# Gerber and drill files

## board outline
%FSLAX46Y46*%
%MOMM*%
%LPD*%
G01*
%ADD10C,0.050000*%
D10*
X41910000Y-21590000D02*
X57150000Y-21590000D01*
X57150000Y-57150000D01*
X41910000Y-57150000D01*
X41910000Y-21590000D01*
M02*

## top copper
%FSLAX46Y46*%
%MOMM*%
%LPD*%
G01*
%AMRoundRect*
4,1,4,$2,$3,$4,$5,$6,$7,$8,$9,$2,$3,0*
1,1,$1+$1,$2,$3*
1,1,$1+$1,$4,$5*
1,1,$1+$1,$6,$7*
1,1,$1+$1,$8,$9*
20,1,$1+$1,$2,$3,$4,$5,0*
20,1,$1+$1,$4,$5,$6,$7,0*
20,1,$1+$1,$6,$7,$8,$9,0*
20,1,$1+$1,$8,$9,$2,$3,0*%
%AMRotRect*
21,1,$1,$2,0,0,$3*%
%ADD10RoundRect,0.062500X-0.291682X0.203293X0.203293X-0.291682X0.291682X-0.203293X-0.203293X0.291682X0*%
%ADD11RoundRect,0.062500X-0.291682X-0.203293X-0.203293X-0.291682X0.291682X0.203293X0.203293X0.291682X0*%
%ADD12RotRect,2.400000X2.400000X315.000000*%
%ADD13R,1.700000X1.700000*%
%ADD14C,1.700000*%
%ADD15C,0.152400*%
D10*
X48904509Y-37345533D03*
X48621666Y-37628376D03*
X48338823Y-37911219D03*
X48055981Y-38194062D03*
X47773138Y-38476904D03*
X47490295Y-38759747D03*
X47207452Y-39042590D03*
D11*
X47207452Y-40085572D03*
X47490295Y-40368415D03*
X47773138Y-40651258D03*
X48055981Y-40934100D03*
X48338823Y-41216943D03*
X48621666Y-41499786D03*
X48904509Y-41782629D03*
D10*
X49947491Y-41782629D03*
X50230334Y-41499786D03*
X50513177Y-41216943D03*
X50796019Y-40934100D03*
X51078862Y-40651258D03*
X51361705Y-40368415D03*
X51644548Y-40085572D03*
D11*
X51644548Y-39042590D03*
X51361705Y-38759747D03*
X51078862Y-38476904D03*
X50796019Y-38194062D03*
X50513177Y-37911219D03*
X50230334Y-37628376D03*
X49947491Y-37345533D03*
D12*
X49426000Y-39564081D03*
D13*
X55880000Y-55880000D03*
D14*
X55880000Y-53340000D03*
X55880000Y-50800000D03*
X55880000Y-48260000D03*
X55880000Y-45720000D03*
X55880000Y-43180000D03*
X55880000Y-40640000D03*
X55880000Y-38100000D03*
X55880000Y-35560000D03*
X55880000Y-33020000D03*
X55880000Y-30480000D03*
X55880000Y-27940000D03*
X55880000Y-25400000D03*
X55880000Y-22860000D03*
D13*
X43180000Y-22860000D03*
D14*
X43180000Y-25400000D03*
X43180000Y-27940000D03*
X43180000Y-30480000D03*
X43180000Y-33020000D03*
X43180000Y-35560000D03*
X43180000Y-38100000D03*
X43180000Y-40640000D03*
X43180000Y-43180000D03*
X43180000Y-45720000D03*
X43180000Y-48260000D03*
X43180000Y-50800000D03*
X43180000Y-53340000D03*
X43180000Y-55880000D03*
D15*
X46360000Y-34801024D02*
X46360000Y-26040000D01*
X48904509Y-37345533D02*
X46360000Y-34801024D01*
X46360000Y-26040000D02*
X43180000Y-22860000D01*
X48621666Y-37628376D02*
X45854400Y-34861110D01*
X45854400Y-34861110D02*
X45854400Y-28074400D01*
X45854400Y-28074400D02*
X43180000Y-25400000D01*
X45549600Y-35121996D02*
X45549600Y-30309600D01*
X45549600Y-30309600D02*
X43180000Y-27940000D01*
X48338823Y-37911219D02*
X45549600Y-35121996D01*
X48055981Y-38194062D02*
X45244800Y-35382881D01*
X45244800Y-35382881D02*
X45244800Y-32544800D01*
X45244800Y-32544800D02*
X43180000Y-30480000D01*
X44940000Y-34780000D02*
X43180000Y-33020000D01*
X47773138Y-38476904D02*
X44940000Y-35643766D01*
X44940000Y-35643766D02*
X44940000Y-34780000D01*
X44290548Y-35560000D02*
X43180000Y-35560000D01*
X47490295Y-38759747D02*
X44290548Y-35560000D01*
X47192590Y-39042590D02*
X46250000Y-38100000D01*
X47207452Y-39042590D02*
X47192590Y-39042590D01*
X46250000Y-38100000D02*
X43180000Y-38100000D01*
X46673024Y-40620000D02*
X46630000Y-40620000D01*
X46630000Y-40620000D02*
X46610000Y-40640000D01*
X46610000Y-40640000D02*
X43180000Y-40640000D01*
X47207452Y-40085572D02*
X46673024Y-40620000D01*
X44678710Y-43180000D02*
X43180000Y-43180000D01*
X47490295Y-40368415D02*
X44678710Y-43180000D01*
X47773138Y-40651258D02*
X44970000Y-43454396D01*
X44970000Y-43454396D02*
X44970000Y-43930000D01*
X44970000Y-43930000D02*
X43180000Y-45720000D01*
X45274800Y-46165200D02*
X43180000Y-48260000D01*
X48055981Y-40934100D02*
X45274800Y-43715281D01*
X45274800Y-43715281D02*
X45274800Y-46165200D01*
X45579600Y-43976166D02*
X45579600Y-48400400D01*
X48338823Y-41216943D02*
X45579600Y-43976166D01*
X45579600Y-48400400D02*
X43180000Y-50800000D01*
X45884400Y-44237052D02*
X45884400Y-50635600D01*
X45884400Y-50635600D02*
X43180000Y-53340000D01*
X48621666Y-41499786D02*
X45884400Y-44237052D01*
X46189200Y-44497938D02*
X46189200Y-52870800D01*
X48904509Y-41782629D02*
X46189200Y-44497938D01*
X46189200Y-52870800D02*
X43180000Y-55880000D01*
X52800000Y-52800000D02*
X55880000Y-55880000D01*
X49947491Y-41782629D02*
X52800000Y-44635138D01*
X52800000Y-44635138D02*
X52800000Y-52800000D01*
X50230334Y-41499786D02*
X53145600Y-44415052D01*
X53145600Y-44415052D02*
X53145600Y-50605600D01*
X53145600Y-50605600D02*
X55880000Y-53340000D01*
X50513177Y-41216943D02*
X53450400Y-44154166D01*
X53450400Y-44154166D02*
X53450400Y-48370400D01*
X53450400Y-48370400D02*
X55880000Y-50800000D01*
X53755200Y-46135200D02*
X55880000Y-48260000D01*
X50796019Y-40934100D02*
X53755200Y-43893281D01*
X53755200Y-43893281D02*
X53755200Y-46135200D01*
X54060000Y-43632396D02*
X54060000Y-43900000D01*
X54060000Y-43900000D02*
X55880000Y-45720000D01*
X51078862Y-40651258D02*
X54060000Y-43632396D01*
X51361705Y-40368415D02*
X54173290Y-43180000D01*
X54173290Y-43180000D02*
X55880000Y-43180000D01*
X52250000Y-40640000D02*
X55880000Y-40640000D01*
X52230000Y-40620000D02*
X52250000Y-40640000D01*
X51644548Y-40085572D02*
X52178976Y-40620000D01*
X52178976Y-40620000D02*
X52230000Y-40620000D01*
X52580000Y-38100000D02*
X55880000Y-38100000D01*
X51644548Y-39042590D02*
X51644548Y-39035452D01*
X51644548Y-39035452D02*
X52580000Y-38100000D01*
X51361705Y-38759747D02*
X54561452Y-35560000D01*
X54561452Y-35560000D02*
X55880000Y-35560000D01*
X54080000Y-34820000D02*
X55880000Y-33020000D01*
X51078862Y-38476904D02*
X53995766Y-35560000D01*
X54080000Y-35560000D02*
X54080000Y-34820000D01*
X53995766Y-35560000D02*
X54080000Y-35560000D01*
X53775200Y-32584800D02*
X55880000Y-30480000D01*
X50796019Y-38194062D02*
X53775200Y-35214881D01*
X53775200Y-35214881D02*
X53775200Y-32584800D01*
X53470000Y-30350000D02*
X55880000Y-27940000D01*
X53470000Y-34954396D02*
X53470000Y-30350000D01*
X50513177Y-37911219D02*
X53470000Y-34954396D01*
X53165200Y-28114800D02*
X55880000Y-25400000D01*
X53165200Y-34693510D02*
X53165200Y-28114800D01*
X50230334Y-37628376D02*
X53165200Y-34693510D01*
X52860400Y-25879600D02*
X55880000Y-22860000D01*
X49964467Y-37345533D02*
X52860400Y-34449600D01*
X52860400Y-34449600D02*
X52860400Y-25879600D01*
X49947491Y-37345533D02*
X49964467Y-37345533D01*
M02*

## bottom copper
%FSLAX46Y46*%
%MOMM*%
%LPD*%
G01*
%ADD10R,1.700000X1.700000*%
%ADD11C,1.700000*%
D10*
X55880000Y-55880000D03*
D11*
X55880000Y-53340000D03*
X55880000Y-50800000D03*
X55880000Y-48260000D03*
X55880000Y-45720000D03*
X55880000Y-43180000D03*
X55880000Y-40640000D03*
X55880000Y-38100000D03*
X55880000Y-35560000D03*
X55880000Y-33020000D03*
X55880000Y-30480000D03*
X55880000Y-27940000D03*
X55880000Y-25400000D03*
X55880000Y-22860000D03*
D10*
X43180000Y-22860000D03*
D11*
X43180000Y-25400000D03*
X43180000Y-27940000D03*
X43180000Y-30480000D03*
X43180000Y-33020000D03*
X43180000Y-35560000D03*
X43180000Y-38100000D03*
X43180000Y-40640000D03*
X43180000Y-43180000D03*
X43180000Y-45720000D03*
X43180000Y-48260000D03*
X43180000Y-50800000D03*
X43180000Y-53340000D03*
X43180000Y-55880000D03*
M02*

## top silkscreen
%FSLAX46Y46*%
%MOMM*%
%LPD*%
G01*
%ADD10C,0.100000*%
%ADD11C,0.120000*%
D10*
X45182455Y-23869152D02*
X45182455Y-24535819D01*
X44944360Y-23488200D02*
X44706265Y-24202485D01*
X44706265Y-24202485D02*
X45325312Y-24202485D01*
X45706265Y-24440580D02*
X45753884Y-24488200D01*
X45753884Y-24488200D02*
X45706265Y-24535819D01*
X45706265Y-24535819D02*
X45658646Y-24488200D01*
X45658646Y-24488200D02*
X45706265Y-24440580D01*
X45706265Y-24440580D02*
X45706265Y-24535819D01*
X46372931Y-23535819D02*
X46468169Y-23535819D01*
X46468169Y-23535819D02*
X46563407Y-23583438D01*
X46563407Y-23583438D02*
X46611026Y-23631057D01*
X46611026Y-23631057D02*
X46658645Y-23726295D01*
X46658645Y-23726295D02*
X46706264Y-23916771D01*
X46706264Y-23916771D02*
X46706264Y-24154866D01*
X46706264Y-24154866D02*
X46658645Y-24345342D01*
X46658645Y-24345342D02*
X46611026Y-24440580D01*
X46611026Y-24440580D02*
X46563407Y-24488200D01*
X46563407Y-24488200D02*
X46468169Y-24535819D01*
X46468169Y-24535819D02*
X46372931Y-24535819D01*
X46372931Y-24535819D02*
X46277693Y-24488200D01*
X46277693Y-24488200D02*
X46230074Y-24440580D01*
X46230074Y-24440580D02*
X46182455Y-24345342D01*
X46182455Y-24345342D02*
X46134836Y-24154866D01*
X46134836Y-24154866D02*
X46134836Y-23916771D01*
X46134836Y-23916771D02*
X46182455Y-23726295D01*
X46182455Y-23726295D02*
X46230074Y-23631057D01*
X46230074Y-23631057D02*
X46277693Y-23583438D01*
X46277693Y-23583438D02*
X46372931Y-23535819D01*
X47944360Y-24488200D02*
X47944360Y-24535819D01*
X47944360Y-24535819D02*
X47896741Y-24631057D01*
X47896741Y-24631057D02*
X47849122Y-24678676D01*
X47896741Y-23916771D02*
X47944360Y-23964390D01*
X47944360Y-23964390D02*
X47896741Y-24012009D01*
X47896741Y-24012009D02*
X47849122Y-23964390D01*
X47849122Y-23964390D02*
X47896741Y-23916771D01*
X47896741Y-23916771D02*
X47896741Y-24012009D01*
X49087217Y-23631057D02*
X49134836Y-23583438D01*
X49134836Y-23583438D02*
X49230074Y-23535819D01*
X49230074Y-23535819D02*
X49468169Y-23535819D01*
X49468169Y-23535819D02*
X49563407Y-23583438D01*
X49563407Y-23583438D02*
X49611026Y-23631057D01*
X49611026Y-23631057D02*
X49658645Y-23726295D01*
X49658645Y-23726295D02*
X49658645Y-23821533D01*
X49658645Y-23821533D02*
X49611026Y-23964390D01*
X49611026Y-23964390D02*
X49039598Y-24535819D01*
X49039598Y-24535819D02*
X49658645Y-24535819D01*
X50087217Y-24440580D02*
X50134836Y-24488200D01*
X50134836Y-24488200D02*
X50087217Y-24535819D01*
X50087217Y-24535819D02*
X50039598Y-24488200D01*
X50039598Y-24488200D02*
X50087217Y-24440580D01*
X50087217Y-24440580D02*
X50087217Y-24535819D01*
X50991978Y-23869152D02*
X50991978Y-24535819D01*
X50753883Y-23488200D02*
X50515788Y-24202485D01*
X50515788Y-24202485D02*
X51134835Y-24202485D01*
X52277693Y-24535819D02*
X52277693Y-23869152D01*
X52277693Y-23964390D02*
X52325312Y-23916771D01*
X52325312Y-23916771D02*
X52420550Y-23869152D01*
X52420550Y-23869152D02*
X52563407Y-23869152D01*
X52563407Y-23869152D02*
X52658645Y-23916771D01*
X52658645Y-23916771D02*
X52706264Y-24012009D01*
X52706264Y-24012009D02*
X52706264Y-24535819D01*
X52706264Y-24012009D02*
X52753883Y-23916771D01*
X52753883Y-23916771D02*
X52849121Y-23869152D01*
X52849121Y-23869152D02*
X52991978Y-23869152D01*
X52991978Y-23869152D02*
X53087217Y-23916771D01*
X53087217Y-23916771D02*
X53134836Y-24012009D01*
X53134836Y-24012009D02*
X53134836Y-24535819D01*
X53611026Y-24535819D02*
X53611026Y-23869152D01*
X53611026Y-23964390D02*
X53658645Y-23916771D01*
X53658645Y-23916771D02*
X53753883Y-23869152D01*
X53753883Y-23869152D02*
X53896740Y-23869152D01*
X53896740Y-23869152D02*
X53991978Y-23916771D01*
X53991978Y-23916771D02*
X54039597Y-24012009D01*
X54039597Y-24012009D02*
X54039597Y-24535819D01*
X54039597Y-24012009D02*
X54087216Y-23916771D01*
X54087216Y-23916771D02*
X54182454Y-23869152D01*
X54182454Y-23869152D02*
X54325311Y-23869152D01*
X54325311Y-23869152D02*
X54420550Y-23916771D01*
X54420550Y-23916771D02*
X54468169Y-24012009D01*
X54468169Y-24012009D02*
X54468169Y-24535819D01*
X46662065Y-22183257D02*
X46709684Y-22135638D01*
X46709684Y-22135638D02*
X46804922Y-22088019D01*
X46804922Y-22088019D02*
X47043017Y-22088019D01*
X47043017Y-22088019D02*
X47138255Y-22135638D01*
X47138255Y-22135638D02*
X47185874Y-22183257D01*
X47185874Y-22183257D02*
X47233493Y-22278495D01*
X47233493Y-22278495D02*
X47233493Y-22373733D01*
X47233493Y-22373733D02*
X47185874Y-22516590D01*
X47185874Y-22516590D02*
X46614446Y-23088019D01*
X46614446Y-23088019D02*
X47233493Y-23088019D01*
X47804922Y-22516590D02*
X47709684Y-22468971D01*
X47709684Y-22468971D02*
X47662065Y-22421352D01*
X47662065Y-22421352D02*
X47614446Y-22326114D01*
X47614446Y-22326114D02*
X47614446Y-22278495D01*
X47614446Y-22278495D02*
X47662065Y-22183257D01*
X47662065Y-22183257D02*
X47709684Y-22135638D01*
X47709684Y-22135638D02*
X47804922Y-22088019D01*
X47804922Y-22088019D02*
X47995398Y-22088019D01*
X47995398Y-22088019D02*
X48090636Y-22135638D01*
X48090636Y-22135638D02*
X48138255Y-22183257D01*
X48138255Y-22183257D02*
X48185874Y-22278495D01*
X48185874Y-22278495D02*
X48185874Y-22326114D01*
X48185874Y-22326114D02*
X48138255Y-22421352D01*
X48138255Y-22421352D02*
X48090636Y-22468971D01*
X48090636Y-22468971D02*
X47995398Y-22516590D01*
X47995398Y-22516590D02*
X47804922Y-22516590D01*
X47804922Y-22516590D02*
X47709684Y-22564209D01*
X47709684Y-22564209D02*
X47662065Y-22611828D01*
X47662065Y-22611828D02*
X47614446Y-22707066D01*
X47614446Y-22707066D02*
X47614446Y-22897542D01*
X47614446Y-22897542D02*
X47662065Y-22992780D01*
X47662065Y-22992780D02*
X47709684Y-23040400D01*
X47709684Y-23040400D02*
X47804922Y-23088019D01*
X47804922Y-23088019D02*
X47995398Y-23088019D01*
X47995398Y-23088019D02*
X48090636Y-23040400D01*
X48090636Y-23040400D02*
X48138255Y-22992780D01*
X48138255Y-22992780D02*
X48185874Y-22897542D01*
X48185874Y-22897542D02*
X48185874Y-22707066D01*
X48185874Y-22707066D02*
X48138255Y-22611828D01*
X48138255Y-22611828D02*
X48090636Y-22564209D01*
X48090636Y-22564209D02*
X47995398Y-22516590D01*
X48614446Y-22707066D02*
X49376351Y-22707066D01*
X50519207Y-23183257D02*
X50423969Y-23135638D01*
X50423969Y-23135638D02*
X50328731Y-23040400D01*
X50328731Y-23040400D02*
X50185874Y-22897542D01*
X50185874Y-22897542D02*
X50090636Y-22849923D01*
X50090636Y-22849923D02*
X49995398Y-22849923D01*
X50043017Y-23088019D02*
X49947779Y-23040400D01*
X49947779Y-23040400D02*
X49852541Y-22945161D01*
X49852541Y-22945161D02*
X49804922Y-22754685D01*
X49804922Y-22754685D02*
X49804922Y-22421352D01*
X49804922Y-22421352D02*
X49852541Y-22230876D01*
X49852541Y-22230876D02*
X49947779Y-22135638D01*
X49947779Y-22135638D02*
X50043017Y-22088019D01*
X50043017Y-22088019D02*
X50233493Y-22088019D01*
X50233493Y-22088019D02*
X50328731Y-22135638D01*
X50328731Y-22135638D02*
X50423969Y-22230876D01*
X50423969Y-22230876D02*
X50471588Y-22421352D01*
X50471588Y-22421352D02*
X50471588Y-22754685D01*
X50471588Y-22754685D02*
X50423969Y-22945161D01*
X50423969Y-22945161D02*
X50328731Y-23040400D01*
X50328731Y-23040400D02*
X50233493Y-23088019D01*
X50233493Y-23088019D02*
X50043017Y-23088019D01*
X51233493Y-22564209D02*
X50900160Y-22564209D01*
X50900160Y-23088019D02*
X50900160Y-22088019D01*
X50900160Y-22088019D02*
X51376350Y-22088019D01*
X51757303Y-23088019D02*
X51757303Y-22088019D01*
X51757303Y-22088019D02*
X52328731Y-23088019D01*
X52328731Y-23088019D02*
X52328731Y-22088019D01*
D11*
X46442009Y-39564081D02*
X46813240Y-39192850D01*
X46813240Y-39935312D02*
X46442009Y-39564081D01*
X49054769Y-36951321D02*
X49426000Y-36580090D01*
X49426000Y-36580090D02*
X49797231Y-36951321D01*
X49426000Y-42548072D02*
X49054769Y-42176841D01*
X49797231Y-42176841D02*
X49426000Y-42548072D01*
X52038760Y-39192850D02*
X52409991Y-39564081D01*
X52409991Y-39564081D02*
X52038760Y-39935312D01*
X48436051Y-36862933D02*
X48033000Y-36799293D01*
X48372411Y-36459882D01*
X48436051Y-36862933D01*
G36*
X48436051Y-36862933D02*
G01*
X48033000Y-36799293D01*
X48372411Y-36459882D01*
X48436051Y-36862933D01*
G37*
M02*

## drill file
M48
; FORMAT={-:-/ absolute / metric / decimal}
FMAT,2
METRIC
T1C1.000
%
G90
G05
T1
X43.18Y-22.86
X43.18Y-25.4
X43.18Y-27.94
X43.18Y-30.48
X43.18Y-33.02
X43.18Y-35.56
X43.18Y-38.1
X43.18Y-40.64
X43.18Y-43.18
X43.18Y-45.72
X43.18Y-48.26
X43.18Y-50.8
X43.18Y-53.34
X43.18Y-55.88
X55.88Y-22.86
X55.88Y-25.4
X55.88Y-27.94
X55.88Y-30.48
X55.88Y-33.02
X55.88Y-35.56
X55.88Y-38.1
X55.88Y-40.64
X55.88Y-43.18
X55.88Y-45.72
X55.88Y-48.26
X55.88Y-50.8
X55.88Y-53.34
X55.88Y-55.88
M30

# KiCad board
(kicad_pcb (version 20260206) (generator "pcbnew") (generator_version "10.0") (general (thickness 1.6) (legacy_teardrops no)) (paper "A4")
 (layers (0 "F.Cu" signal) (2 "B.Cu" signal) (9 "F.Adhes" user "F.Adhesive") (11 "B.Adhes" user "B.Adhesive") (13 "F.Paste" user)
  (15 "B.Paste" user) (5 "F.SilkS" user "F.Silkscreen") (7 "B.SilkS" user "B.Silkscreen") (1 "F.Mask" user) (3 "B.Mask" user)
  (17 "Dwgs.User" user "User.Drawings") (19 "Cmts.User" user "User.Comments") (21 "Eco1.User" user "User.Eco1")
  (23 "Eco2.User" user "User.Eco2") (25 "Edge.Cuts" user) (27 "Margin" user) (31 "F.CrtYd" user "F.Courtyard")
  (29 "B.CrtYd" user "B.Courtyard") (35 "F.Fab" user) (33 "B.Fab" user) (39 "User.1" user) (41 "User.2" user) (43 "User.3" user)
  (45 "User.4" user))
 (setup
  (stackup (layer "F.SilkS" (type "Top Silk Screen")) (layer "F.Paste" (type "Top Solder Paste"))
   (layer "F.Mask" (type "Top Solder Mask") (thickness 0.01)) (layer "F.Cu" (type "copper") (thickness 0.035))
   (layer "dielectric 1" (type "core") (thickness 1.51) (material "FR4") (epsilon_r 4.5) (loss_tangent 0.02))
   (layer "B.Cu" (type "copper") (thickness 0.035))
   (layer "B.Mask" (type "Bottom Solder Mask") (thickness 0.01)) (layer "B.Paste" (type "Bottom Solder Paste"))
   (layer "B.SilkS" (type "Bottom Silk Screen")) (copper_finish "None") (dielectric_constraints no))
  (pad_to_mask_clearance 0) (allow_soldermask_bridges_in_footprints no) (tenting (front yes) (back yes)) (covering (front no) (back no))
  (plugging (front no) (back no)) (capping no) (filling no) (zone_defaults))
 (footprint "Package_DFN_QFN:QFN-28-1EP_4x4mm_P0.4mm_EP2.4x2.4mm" (layer "F.Cu") (at 49.426 39.564081 -45)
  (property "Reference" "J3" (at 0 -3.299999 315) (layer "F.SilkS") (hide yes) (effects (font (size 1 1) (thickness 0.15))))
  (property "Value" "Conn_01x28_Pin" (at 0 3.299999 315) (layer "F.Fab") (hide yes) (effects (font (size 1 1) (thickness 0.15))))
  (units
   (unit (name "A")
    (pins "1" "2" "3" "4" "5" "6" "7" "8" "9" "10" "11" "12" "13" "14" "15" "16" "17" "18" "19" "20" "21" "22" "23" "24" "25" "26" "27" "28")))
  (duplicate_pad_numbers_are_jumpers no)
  (fp_line (start -2.11 2.11) (end -2.11 1.585) (stroke (width 0.12) (type solid)) (layer "F.SilkS"))
  (fp_line (start -1.585 2.11) (end -2.11 2.11) (stroke (width 0.12) (type solid)) (layer "F.SilkS"))
  (fp_line (start -2.11 -1.585) (end -2.11 -2.11) (stroke (width 0.12) (type solid)) (layer "F.SilkS"))
  (fp_line (start -2.11 -2.11) (end -1.585 -2.11) (stroke (width 0.12) (type solid)) (layer "F.SilkS"))
  (fp_line (start 2.11 2.11) (end 1.585 2.11) (stroke (width 0.12) (type solid)) (layer "F.SilkS"))
  (fp_line (start 2.11 1.585) (end 2.11 2.11) (stroke (width 0.12) (type solid)) (layer "F.SilkS"))
  (fp_line (start 1.585 -2.11) (end 2.11 -2.11) (stroke (width 0.12) (type solid)) (layer "F.SilkS"))
  (fp_line (start 2.11 -2.11) (end 2.11 -1.585) (stroke (width 0.12) (type solid)) (layer "F.SilkS"))
  (fp_poly (pts (xy -2.61 -1.21) (xy -2.94 -0.970001) (xy -2.94 -1.45)) (stroke (width 0.12) (type solid)) (fill yes) (layer "F.SilkS"))
  (pad "" smd roundrect (at -0.6 -0.6 315) (size 0.97 0.97) (layers "F.Paste") (roundrect_rratio 0.25))
  (pad "" smd roundrect (at -0.6 0.6 315) (size 0.97 0.97) (layers "F.Paste") (roundrect_rratio 0.25))
  (pad "" smd roundrect (at 0.6 -0.6 315) (size 0.97 0.97) (layers "F.Paste") (roundrect_rratio 0.25))
  (pad "" smd roundrect (at 0.6 0.6 315) (size 0.97 0.97) (layers "F.Paste") (roundrect_rratio 0.25))
  (pad "1" smd roundrect (at -1.9375 -1.200001 315) (size 0.825 0.25) (layers "F.Cu" "F.Mask" "F.Paste") (roundrect_rratio 0.25)
   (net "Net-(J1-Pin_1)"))
  (pad "2" smd roundrect (at -1.9375 -0.8 315) (size 0.825 0.25) (layers "F.Cu" "F.Mask" "F.Paste") (roundrect_rratio 0.25)
   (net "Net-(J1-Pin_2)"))
  (pad "3" smd roundrect (at -1.9375 -0.4 315) (size 0.825 0.25) (layers "F.Cu" "F.Mask" "F.Paste") (roundrect_rratio 0.25)
   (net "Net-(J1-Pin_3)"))
  (pad "4" smd roundrect (at -1.937499 0 315) (size 0.825 0.25) (layers "F.Cu" "F.Mask" "F.Paste") (roundrect_rratio 0.25)
   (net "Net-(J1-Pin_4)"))
  (pad "5" smd roundrect (at -1.9375 0.4 315) (size 0.825 0.25) (layers "F.Cu" "F.Mask" "F.Paste") (roundrect_rratio 0.25)
   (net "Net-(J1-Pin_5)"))
  (pad "6" smd roundrect (at -1.9375 0.8 315) (size 0.825 0.25) (layers "F.Cu" "F.Mask" "F.Paste") (roundrect_rratio 0.25)
   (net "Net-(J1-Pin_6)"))
  (pad "7" smd roundrect (at -1.9375 1.200001 315) (size 0.825 0.25) (layers "F.Cu" "F.Mask" "F.Paste") (roundrect_rratio 0.25)
   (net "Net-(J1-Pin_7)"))
  (pad "8" smd roundrect (at -1.200001 1.9375 315) (size 0.25 0.825) (layers "F.Cu" "F.Mask" "F.Paste") (roundrect_rratio 0.25)
   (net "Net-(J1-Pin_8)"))
  (pad "9" smd roundrect (at -0.8 1.9375 315) (size 0.25 0.825) (layers "F.Cu" "F.Mask" "F.Paste") (roundrect_rratio 0.25)
   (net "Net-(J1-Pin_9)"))
  (pad "10" smd roundrect (at -0.4 1.9375 315) (size 0.25 0.825) (layers "F.Cu" "F.Mask" "F.Paste") (roundrect_rratio 0.25)
   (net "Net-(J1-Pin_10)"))
  (pad "11" smd roundrect (at 0 1.937499 315) (size 0.25 0.825) (layers "F.Cu" "F.Mask" "F.Paste") (roundrect_rratio 0.25)
   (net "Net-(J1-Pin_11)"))
  (pad "12" smd roundrect (at 0.4 1.9375 315) (size 0.25 0.825) (layers "F.Cu" "F.Mask" "F.Paste") (roundrect_rratio 0.25)
   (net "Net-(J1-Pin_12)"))
  (pad "13" smd roundrect (at 0.8 1.9375 315) (size 0.25 0.825) (layers "F.Cu" "F.Mask" "F.Paste") (roundrect_rratio 0.25)
   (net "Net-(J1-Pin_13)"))
  (pad "14" smd roundrect (at 1.200001 1.9375 315) (size 0.25 0.825) (layers "F.Cu" "F.Mask" "F.Paste") (roundrect_rratio 0.25)
   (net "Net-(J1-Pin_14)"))
  (pad "15" smd roundrect (at 1.9375 1.200001 315) (size 0.825 0.25) (layers "F.Cu" "F.Mask" "F.Paste") (roundrect_rratio 0.25)
   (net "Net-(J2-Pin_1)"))
  (pad "16" smd roundrect (at 1.9375 0.8 315) (size 0.825 0.25) (layers "F.Cu" "F.Mask" "F.Paste") (roundrect_rratio 0.25)
   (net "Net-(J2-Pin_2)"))
  (pad "17" smd roundrect (at 1.9375 0.4 315) (size 0.825 0.25) (layers "F.Cu" "F.Mask" "F.Paste") (roundrect_rratio 0.25)
   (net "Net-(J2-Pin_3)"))
  (pad "18" smd roundrect (at 1.937499 0 315) (size 0.825 0.25) (layers "F.Cu" "F.Mask" "F.Paste") (roundrect_rratio 0.25)
   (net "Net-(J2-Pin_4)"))
  (pad "19" smd roundrect (at 1.9375 -0.4 315) (size 0.825 0.25) (layers "F.Cu" "F.Mask" "F.Paste") (roundrect_rratio 0.25)
   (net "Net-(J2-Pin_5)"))
  (pad "20" smd roundrect (at 1.9375 -0.8 315) (size 0.825 0.25) (layers "F.Cu" "F.Mask" "F.Paste") (roundrect_rratio 0.25)
   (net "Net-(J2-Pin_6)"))
  (pad "21" smd roundrect (at 1.9375 -1.200001 315) (size 0.825 0.25) (layers "F.Cu" "F.Mask" "F.Paste") (roundrect_rratio 0.25)
   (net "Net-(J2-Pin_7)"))
  (pad "22" smd roundrect (at 1.200001 -1.9375 315) (size 0.25 0.825) (layers "F.Cu" "F.Mask" "F.Paste") (roundrect_rratio 0.25)
   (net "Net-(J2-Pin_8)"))
  (pad "23" smd roundrect (at 0.8 -1.9375 315) (size 0.25 0.825) (layers "F.Cu" "F.Mask" "F.Paste") (roundrect_rratio 0.25)
   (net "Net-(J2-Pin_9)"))
  (pad "24" smd roundrect (at 0.4 -1.9375 315) (size 0.25 0.825) (layers "F.Cu" "F.Mask" "F.Paste") (roundrect_rratio 0.25)
   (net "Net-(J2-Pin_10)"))
  (pad "25" smd roundrect (at 0 -1.937499 315) (size 0.25 0.825) (layers "F.Cu" "F.Mask" "F.Paste") (roundrect_rratio 0.25)
   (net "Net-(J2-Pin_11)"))
  (pad "26" smd roundrect (at -0.4 -1.9375 315) (size 0.25 0.825) (layers "F.Cu" "F.Mask" "F.Paste") (roundrect_rratio 0.25)
   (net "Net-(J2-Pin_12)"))
  (pad "27" smd roundrect (at -0.8 -1.9375 315) (size 0.25 0.825) (layers "F.Cu" "F.Mask" "F.Paste") (roundrect_rratio 0.25)
   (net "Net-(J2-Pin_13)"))
  (pad "28" smd roundrect (at -1.200001 -1.9375 315) (size 0.25 0.825) (layers "F.Cu" "F.Mask" "F.Paste") (roundrect_rratio 0.25)
   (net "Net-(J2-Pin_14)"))
  (pad "29" smd rect (at 0 0 315) (size 2.4 2.4) (layers "F.Cu" "F.Mask") (zone_connect 2)))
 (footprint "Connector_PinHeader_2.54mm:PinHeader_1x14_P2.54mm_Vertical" (layer "B.Cu") (at 55.88 55.88)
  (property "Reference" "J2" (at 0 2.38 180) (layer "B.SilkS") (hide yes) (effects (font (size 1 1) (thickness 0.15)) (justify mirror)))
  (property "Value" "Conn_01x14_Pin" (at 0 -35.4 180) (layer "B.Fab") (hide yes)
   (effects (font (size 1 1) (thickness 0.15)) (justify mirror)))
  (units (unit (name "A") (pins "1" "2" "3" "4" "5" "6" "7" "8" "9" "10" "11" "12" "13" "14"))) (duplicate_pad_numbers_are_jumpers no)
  (pad "1" thru_hole rect (at 0 0) (size 1.7 1.7) (drill 1) (layers "*.Cu" "*.Mask") (remove_unused_layers no) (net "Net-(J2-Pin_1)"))
  (pad "2" thru_hole circle (at 0 -2.54) (size 1.7 1.7) (drill 1) (layers "*.Cu" "*.Mask") (remove_unused_layers no) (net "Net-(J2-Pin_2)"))
  (pad "3" thru_hole circle (at 0 -5.08) (size 1.7 1.7) (drill 1) (layers "*.Cu" "*.Mask") (remove_unused_layers no) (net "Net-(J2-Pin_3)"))
  (pad "4" thru_hole circle (at 0 -7.62) (size 1.7 1.7) (drill 1) (layers "*.Cu" "*.Mask") (remove_unused_layers no) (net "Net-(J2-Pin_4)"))
  (pad "5" thru_hole circle (at 0 -10.16) (size 1.7 1.7) (drill 1) (layers "*.Cu" "*.Mask") (remove_unused_layers no) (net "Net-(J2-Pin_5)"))
  (pad "6" thru_hole circle (at 0 -12.7) (size 1.7 1.7) (drill 1) (layers "*.Cu" "*.Mask") (remove_unused_layers no) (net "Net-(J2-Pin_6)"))
  (pad "7" thru_hole circle (at 0 -15.24) (size 1.7 1.7) (drill 1) (layers "*.Cu" "*.Mask") (remove_unused_layers no) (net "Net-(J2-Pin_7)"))
  (pad "8" thru_hole circle (at 0 -17.78) (size 1.7 1.7) (drill 1) (layers "*.Cu" "*.Mask") (remove_unused_layers no) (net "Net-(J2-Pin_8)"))
  (pad "9" thru_hole circle (at 0 -20.32) (size 1.7 1.7) (drill 1) (layers "*.Cu" "*.Mask") (remove_unused_layers no) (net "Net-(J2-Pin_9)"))
  (pad "10" thru_hole circle (at 0 -22.86) (size 1.7 1.7) (drill 1) (layers "*.Cu" "*.Mask") (remove_unused_layers no)
   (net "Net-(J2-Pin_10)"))
  (pad "11" thru_hole circle (at 0 -25.4) (size 1.7 1.7) (drill 1) (layers "*.Cu" "*.Mask") (remove_unused_layers no)
   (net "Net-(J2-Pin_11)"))
  (pad "12" thru_hole circle (at 0 -27.94) (size 1.7 1.7) (drill 1) (layers "*.Cu" "*.Mask") (remove_unused_layers no)
   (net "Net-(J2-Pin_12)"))
  (pad "13" thru_hole circle (at 0 -30.48) (size 1.7 1.7) (drill 1) (layers "*.Cu" "*.Mask") (remove_unused_layers no)
   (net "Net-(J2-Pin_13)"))
  (pad "14" thru_hole circle (at 0 -33.02) (size 1.7 1.7) (drill 1) (layers "*.Cu" "*.Mask") (remove_unused_layers no)
   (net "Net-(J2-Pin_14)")))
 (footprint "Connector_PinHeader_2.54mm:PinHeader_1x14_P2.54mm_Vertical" (layer "B.Cu") (at 43.18 22.86 180)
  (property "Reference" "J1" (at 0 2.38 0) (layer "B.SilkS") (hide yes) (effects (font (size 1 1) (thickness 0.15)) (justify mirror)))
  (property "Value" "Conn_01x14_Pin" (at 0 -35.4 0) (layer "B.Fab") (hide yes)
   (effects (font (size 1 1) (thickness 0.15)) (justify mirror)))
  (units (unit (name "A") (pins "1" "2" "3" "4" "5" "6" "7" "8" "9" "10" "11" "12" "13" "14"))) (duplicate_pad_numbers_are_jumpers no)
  (pad "1" thru_hole rect (at 0 0 180) (size 1.7 1.7) (drill 1) (layers "*.Cu" "*.Mask") (remove_unused_layers no) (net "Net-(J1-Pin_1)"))
  (pad "2" thru_hole circle (at 0 -2.54 180) (size 1.7 1.7) (drill 1) (layers "*.Cu" "*.Mask") (remove_unused_layers no)
   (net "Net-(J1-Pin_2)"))
  (pad "3" thru_hole circle (at 0 -5.08 180) (size 1.7 1.7) (drill 1) (layers "*.Cu" "*.Mask") (remove_unused_layers no)
   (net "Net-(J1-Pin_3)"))
  (pad "4" thru_hole circle (at 0 -7.62 180) (size 1.7 1.7) (drill 1) (layers "*.Cu" "*.Mask") (remove_unused_layers no)
   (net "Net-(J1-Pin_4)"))
  (pad "5" thru_hole circle (at 0 -10.16 180) (size 1.7 1.7) (drill 1) (layers "*.Cu" "*.Mask") (remove_unused_layers no)
   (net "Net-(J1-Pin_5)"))
  (pad "6" thru_hole circle (at 0 -12.7 180) (size 1.7 1.7) (drill 1) (layers "*.Cu" "*.Mask") (remove_unused_layers no)
   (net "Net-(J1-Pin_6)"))
  (pad "7" thru_hole circle (at 0 -15.24 180) (size 1.7 1.7) (drill 1) (layers "*.Cu" "*.Mask") (remove_unused_layers no)
   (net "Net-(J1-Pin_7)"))
  (pad "8" thru_hole circle (at 0 -17.78 180) (size 1.7 1.7) (drill 1) (layers "*.Cu" "*.Mask") (remove_unused_layers no)
   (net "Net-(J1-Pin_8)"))
  (pad "9" thru_hole circle (at 0 -20.32 180) (size 1.7 1.7) (drill 1) (layers "*.Cu" "*.Mask") (remove_unused_layers no)
   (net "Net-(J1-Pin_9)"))
  (pad "10" thru_hole circle (at 0 -22.86 180) (size 1.7 1.7) (drill 1) (layers "*.Cu" "*.Mask") (remove_unused_layers no)
   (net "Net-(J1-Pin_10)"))
  (pad "11" thru_hole circle (at 0 -25.4 180) (size 1.7 1.7) (drill 1) (layers "*.Cu" "*.Mask") (remove_unused_layers no)
   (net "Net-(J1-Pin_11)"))
  (pad "12" thru_hole circle (at 0 -27.94 180) (size 1.7 1.7) (drill 1) (layers "*.Cu" "*.Mask") (remove_unused_layers no)
   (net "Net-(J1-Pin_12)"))
  (pad "13" thru_hole circle (at 0 -30.48 180) (size 1.7 1.7) (drill 1) (layers "*.Cu" "*.Mask") (remove_unused_layers no)
   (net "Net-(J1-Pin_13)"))
  (pad "14" thru_hole circle (at 0 -33.02 180) (size 1.7 1.7) (drill 1) (layers "*.Cu" "*.Mask") (remove_unused_layers no)
   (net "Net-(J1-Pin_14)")))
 (gr_rect (start 41.91 21.59) (end 57.15 57.15) (stroke (width 0.05) (type default)) (fill no) (layer "Edge.Cuts"))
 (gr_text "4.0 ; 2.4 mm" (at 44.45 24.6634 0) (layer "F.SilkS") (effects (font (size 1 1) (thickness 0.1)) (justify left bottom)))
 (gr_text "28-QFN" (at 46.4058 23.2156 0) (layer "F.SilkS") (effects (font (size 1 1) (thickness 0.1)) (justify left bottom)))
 (segment (start 46.36 34.801024) (end 46.36 26.04) (width 0.1524) (layer "F.Cu") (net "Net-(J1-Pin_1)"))
 (segment (start 48.904509 37.345533) (end 46.36 34.801024) (width 0.1524) (layer "F.Cu") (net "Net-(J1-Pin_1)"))
 (segment (start 46.36 26.04) (end 43.18 22.86) (width 0.1524) (layer "F.Cu") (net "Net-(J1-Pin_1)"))
 (segment (start 48.621666 37.628376) (end 45.8544 34.86111) (width 0.1524) (layer "F.Cu") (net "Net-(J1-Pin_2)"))
 (segment (start 45.8544 34.86111) (end 45.8544 28.0744) (width 0.1524) (layer "F.Cu") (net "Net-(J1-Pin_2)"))
 (segment (start 45.8544 28.0744) (end 43.18 25.4) (width 0.1524) (layer "F.Cu") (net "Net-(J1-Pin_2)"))
 (segment (start 45.5496 35.121996) (end 45.5496 30.3096) (width 0.1524) (layer "F.Cu") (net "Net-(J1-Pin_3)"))
 (segment (start 45.5496 30.3096) (end 43.18 27.94) (width 0.1524) (layer "F.Cu") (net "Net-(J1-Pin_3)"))
 (segment (start 48.338823 37.911219) (end 45.5496 35.121996) (width 0.1524) (layer "F.Cu") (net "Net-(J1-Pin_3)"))
 (segment (start 48.055981 38.194062) (end 45.2448 35.382881) (width 0.1524) (layer "F.Cu") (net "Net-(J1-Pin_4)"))
 (segment (start 45.2448 35.382881) (end 45.2448 32.5448) (width 0.1524) (layer "F.Cu") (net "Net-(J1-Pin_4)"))
 (segment (start 45.2448 32.5448) (end 43.18 30.48) (width 0.1524) (layer "F.Cu") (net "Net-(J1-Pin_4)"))
 (segment (start 44.94 34.78) (end 43.18 33.02) (width 0.1524) (layer "F.Cu") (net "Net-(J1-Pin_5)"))
 (segment (start 47.773138 38.476904) (end 44.94 35.643766) (width 0.1524) (layer "F.Cu") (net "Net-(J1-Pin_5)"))
 (segment (start 44.94 35.643766) (end 44.94 34.78) (width 0.1524) (layer "F.Cu") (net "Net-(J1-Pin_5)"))
 (segment (start 44.290548 35.56) (end 43.18 35.56) (width 0.1524) (layer "F.Cu") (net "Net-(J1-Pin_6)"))
 (segment (start 47.490295 38.759747) (end 44.290548 35.56) (width 0.1524) (layer "F.Cu") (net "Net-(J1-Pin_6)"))
 (segment (start 47.19259 39.04259) (end 46.25 38.1) (width 0.1524) (layer "F.Cu") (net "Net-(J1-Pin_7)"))
 (segment (start 47.207452 39.04259) (end 47.19259 39.04259) (width 0.1524) (layer "F.Cu") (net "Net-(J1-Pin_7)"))
 (segment (start 46.25 38.1) (end 43.18 38.1) (width 0.1524) (layer "F.Cu") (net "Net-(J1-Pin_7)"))
 (segment (start 46.673024 40.62) (end 46.63 40.62) (width 0.1524) (layer "F.Cu") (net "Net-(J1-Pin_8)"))
 (segment (start 46.63 40.62) (end 46.61 40.64) (width 0.1524) (layer "F.Cu") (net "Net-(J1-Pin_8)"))
 (segment (start 46.61 40.64) (end 43.18 40.64) (width 0.1524) (layer "F.Cu") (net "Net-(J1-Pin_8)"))
 (segment (start 47.207452 40.085572) (end 46.673024 40.62) (width 0.1524) (layer "F.Cu") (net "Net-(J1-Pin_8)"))
 (segment (start 44.67871 43.18) (end 43.18 43.18) (width 0.1524) (layer "F.Cu") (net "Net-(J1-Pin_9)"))
 (segment (start 47.490295 40.368415) (end 44.67871 43.18) (width 0.1524) (layer "F.Cu") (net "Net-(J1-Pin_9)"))
 (segment (start 47.773138 40.651258) (end 44.97 43.454396) (width 0.1524) (layer "F.Cu") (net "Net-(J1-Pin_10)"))
 (segment (start 44.97 43.454396) (end 44.97 43.93) (width 0.1524) (layer "F.Cu") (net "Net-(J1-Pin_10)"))
 (segment (start 44.97 43.93) (end 43.18 45.72) (width 0.1524) (layer "F.Cu") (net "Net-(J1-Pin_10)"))
 (segment (start 45.2748 46.1652) (end 43.18 48.26) (width 0.1524) (layer "F.Cu") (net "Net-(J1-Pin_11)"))
 (segment (start 48.055981 40.9341) (end 45.2748 43.715281) (width 0.1524) (layer "F.Cu") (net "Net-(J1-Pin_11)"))
 (segment (start 45.2748 43.715281) (end 45.2748 46.1652) (width 0.1524) (layer "F.Cu") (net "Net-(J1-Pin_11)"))
 (segment (start 45.5796 43.976166) (end 45.5796 48.4004) (width 0.1524) (layer "F.Cu") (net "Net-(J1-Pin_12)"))
 (segment (start 48.338823 41.216943) (end 45.5796 43.976166) (width 0.1524) (layer "F.Cu") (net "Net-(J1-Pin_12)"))
 (segment (start 45.5796 48.4004) (end 43.18 50.8) (width 0.1524) (layer "F.Cu") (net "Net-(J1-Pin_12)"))
 (segment (start 45.8844 44.237052) (end 45.8844 50.6356) (width 0.1524) (layer "F.Cu") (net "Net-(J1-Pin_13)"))
 (segment (start 45.8844 50.6356) (end 43.18 53.34) (width 0.1524) (layer "F.Cu") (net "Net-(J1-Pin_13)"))
 (segment (start 48.621666 41.499786) (end 45.8844 44.237052) (width 0.1524) (layer "F.Cu") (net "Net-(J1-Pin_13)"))
 (segment (start 46.1892 44.497938) (end 46.1892 52.8708) (width 0.1524) (layer "F.Cu") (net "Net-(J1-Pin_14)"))
 (segment (start 48.904509 41.782629) (end 46.1892 44.497938) (width 0.1524) (layer "F.Cu") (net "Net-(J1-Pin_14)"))
 (segment (start 46.1892 52.8708) (end 43.18 55.88) (width 0.1524) (layer "F.Cu") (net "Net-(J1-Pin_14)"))
 (segment (start 52.8 52.8) (end 55.88 55.88) (width 0.1524) (layer "F.Cu") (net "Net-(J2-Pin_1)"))
 (segment (start 49.947491 41.782629) (end 52.8 44.635138) (width 0.1524) (layer "F.Cu") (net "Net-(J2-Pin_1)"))
 (segment (start 52.8 44.635138) (end 52.8 52.8) (width 0.1524) (layer "F.Cu") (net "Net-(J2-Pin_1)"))
 (segment (start 50.230334 41.499786) (end 53.1456 44.415052) (width 0.1524) (layer "F.Cu") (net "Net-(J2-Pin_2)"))
 (segment (start 53.1456 44.415052) (end 53.1456 50.6056) (width 0.1524) (layer "F.Cu") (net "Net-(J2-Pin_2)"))
 (segment (start 53.1456 50.6056) (end 55.88 53.34) (width 0.1524) (layer "F.Cu") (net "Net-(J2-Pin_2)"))
 (segment (start 50.513177 41.216943) (end 53.4504 44.154166) (width 0.1524) (layer "F.Cu") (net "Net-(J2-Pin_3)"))
 (segment (start 53.4504 44.154166) (end 53.4504 48.3704) (width 0.1524) (layer "F.Cu") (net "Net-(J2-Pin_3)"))
 (segment (start 53.4504 48.3704) (end 55.88 50.8) (width 0.1524) (layer "F.Cu") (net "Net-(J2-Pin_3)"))
 (segment (start 53.7552 46.1352) (end 55.88 48.26) (width 0.1524) (layer "F.Cu") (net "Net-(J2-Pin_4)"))
 (segment (start 50.796019 40.9341) (end 53.7552 43.893281) (width 0.1524) (layer "F.Cu") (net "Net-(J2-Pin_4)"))
 (segment (start 53.7552 43.893281) (end 53.7552 46.1352) (width 0.1524) (layer "F.Cu") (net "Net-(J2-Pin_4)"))
 (segment (start 54.06 43.632396) (end 54.06 43.9) (width 0.1524) (layer "F.Cu") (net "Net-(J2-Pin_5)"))
 (segment (start 54.06 43.9) (end 55.88 45.72) (width 0.1524) (layer "F.Cu") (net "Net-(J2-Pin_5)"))
 (segment (start 51.078862 40.651258) (end 54.06 43.632396) (width 0.1524) (layer "F.Cu") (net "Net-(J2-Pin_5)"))
 (segment (start 51.361705 40.368415) (end 54.17329 43.18) (width 0.1524) (layer "F.Cu") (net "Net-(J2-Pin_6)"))
 (segment (start 54.17329 43.18) (end 55.88 43.18) (width 0.1524) (layer "F.Cu") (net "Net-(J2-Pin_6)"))
 (segment (start 52.25 40.64) (end 55.88 40.64) (width 0.1524) (layer "F.Cu") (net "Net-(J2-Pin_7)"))
 (segment (start 52.23 40.62) (end 52.25 40.64) (width 0.1524) (layer "F.Cu") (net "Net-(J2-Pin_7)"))
 (segment (start 51.644548 40.085572) (end 52.178976 40.62) (width 0.1524) (layer "F.Cu") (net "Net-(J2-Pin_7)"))
 (segment (start 52.178976 40.62) (end 52.23 40.62) (width 0.1524) (layer "F.Cu") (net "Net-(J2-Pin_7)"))
 (segment (start 52.58 38.1) (end 55.88 38.1) (width 0.1524) (layer "F.Cu") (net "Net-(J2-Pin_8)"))
 (segment (start 51.644548 39.04259) (end 51.644548 39.035452) (width 0.1524) (layer "F.Cu") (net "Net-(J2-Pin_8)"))
 (segment (start 51.644548 39.035452) (end 52.58 38.1) (width 0.1524) (layer "F.Cu") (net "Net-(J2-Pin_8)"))
 (segment (start 51.361705 38.759747) (end 54.561452 35.56) (width 0.1524) (layer "F.Cu") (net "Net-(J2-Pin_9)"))
 (segment (start 54.561452 35.56) (end 55.88 35.56) (width 0.1524) (layer "F.Cu") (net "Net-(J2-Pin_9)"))
 (segment (start 54.08 34.82) (end 55.88 33.02) (width 0.1524) (layer "F.Cu") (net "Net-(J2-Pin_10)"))
 (segment (start 51.078862 38.476904) (end 53.995766 35.56) (width 0.1524) (layer "F.Cu") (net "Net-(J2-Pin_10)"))
 (segment (start 54.08 35.56) (end 54.08 34.82) (width 0.1524) (layer "F.Cu") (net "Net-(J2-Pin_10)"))
 (segment (start 53.995766 35.56) (end 54.08 35.56) (width 0.1524) (layer "F.Cu") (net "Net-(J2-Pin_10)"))
 (segment (start 53.7752 32.5848) (end 55.88 30.48) (width 0.1524) (layer "F.Cu") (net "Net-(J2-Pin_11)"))
 (segment (start 50.796019 38.194062) (end 53.7752 35.214881) (width 0.1524) (layer "F.Cu") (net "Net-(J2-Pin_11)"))
 (segment (start 53.7752 35.214881) (end 53.7752 32.5848) (width 0.1524) (layer "F.Cu") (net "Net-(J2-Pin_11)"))
 (segment (start 53.47 30.35) (end 55.88 27.94) (width 0.1524) (layer "F.Cu") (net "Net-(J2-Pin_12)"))
 (segment (start 53.47 34.954396) (end 53.47 30.35) (width 0.1524) (layer "F.Cu") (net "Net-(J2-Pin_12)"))
 (segment (start 50.513177 37.911219) (end 53.47 34.954396) (width 0.1524) (layer "F.Cu") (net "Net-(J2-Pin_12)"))
 (segment (start 53.1652 28.1148) (end 55.88 25.4) (width 0.1524) (layer "F.Cu") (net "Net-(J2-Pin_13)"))
 (segment (start 53.1652 34.69351) (end 53.1652 28.1148) (width 0.1524) (layer "F.Cu") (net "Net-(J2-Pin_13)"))
 (segment (start 50.230334 37.628376) (end 53.1652 34.69351) (width 0.1524) (layer "F.Cu") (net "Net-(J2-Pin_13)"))
 (segment (start 52.8604 25.8796) (end 55.88 22.86) (width 0.1524) (layer "F.Cu") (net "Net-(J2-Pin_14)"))
 (segment (start 49.964467 37.345533) (end 52.8604 34.4496) (width 0.1524) (layer "F.Cu") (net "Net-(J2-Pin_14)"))
 (segment (start 52.8604 34.4496) (end 52.8604 25.8796) (width 0.1524) (layer "F.Cu") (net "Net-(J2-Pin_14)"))
 (segment (start 49.947491 37.345533) (end 49.964467 37.345533) (width 0.1524) (layer "F.Cu") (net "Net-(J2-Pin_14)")))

